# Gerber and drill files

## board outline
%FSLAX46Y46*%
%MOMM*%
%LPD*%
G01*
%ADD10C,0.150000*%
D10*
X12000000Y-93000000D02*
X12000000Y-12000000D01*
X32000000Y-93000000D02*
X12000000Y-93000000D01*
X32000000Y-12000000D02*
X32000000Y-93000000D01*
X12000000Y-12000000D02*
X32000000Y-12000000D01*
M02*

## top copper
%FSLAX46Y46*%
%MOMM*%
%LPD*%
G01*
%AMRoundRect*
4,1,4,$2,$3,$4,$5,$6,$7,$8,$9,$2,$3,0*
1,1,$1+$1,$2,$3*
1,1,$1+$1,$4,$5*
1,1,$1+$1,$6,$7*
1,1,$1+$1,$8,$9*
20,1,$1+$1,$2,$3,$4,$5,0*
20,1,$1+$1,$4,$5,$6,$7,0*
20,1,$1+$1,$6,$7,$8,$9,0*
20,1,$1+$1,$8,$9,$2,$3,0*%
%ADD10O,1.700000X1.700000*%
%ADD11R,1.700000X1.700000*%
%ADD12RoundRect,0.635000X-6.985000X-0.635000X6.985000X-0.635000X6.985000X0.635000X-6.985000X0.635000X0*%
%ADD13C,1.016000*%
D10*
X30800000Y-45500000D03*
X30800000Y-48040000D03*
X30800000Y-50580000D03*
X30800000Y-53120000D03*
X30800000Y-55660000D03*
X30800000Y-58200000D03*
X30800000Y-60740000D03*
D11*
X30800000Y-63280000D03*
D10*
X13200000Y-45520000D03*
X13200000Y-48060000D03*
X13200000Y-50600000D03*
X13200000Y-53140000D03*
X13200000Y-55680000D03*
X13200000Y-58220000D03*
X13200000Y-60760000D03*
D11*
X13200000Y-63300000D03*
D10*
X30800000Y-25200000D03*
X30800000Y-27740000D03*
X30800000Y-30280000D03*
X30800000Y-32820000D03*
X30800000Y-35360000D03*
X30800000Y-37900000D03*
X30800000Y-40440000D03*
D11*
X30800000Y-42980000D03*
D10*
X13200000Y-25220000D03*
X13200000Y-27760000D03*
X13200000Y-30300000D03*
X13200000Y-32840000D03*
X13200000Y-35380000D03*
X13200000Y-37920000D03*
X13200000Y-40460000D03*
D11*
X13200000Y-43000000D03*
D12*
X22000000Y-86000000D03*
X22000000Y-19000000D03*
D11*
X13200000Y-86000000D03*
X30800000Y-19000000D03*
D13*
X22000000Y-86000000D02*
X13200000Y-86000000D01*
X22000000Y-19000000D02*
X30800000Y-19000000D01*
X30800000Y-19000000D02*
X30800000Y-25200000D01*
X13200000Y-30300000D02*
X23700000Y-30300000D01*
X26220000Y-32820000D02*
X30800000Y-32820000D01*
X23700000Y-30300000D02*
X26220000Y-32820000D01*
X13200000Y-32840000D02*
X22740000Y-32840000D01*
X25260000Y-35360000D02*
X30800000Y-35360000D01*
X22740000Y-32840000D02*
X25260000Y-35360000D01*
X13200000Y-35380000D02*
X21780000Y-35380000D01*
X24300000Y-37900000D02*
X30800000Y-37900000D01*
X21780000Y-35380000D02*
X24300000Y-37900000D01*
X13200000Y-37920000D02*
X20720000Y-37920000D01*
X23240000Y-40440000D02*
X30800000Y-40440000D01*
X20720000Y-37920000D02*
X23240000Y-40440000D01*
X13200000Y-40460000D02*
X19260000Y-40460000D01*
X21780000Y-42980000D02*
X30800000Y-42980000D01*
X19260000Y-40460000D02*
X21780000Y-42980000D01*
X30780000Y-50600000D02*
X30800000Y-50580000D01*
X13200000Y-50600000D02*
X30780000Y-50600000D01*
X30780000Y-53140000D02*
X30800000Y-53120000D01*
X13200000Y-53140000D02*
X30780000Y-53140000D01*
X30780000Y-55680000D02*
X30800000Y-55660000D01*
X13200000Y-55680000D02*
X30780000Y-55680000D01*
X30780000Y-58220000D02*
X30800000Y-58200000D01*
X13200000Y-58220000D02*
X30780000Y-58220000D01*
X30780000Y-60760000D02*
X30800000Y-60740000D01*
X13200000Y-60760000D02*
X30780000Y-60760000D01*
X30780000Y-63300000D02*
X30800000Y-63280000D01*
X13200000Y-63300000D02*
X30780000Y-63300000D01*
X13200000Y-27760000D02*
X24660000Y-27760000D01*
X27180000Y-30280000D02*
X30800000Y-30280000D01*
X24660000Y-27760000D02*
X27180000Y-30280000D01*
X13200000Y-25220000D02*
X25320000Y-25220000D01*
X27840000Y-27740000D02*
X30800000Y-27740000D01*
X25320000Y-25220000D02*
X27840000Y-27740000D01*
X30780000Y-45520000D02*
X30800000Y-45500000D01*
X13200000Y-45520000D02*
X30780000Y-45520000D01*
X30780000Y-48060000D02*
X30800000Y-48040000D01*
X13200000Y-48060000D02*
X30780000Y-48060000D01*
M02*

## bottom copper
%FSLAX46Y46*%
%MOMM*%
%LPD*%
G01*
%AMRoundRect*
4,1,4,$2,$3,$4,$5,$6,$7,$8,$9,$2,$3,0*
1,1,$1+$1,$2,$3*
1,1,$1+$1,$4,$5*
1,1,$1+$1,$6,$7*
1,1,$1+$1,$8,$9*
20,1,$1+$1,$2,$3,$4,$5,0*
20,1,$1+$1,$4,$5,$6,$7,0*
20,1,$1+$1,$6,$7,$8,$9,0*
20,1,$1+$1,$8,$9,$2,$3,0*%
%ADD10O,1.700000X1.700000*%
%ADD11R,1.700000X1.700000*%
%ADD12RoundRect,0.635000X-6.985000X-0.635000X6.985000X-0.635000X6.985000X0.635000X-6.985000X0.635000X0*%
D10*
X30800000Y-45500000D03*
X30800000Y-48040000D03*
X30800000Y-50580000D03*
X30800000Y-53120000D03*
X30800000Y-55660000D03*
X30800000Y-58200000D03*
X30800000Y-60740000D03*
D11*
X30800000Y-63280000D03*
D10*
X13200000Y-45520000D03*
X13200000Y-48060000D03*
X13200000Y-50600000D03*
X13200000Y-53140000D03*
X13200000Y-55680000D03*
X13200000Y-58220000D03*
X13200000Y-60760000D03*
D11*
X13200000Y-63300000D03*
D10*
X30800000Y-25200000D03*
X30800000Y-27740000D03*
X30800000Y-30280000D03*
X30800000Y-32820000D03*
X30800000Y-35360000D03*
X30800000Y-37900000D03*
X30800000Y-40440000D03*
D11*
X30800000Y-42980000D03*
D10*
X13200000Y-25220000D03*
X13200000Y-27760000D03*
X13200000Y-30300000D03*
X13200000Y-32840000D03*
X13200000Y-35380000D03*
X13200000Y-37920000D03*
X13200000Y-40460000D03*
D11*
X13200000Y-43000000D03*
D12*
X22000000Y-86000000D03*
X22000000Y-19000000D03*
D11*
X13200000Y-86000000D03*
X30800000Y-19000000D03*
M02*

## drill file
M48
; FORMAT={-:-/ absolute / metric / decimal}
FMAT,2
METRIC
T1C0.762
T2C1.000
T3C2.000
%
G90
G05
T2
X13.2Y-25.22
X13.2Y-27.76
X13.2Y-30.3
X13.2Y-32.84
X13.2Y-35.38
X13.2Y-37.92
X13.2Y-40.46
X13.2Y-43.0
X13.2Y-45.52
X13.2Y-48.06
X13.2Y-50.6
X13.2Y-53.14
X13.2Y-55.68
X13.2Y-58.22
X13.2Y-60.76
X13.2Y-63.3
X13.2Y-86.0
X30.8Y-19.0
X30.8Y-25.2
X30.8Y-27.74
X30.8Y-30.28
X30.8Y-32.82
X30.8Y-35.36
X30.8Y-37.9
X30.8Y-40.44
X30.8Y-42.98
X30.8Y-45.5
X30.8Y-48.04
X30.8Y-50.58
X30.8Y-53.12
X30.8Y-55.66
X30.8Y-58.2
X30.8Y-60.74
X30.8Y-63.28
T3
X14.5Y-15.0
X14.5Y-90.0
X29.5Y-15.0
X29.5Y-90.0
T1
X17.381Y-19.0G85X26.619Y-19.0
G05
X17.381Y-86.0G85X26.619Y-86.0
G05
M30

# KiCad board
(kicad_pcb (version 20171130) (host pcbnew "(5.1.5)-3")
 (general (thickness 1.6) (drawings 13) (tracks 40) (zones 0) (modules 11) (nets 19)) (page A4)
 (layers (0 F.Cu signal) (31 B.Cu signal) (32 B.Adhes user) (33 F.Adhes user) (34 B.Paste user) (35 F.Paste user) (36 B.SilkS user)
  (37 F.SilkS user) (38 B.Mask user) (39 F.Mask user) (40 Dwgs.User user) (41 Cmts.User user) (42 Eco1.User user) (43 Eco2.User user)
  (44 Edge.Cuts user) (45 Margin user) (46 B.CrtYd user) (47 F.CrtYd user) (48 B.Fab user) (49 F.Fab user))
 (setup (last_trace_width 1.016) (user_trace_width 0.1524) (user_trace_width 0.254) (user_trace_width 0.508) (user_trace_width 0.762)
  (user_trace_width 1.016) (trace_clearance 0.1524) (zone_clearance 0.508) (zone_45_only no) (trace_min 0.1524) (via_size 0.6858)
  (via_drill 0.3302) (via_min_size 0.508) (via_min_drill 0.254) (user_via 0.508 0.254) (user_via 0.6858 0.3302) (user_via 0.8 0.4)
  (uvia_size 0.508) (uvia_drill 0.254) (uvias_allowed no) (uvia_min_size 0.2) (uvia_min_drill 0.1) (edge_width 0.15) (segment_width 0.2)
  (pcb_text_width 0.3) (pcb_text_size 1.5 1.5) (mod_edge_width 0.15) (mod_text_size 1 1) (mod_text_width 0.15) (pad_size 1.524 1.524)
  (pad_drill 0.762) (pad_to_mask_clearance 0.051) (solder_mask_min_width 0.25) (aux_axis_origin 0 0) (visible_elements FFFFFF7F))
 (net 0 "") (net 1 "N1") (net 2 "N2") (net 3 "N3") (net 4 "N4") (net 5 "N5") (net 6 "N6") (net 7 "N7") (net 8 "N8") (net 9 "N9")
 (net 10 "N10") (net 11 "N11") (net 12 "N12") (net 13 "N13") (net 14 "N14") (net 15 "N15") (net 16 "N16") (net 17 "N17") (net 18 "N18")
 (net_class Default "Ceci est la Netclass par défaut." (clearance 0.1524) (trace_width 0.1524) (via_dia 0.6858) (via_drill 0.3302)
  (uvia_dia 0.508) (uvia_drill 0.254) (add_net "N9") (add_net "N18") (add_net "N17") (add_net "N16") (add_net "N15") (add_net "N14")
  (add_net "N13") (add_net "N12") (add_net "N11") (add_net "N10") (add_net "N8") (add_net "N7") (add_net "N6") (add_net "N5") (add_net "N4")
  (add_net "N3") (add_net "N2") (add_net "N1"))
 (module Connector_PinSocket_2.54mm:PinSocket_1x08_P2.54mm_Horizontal (layer F.Cu) (at 30.8 63.28 180)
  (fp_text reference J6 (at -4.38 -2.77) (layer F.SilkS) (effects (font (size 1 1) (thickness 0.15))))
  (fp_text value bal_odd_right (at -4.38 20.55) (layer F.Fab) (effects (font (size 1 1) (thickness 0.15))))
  (pad 8 thru_hole oval (at 0 17.78 180) (size 1.7 1.7) (drill 1) (layers *.Cu *.Mask) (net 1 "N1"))
  (pad 7 thru_hole oval (at 0 15.24 180) (size 1.7 1.7) (drill 1) (layers *.Cu *.Mask) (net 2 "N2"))
  (pad 6 thru_hole oval (at 0 12.7 180) (size 1.7 1.7) (drill 1) (layers *.Cu *.Mask) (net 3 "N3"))
  (pad 5 thru_hole oval (at 0 10.16 180) (size 1.7 1.7) (drill 1) (layers *.Cu *.Mask) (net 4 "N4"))
  (pad 4 thru_hole oval (at 0 7.62 180) (size 1.7 1.7) (drill 1) (layers *.Cu *.Mask) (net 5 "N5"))
  (pad 3 thru_hole oval (at 0 5.08 180) (size 1.7 1.7) (drill 1) (layers *.Cu *.Mask) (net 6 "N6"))
  (pad 2 thru_hole oval (at 0 2.54 180) (size 1.7 1.7) (drill 1) (layers *.Cu *.Mask) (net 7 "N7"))
  (pad 1 thru_hole rect (at 0 0 180) (size 1.7 1.7) (drill 1) (layers *.Cu *.Mask) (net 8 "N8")))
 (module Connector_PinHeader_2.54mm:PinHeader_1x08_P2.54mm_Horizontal (layer F.Cu) (at 13.2 63.3 180)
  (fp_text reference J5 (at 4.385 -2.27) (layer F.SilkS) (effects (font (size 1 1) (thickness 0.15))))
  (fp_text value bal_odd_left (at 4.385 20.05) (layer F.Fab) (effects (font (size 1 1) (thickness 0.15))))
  (pad 8 thru_hole oval (at 0 17.78 180) (size 1.7 1.7) (drill 1) (layers *.Cu *.Mask) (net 1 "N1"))
  (pad 7 thru_hole oval (at 0 15.24 180) (size 1.7 1.7) (drill 1) (layers *.Cu *.Mask) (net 2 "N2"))
  (pad 6 thru_hole oval (at 0 12.7 180) (size 1.7 1.7) (drill 1) (layers *.Cu *.Mask) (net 3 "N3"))
  (pad 5 thru_hole oval (at 0 10.16 180) (size 1.7 1.7) (drill 1) (layers *.Cu *.Mask) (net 4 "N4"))
  (pad 4 thru_hole oval (at 0 7.62 180) (size 1.7 1.7) (drill 1) (layers *.Cu *.Mask) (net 5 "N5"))
  (pad 3 thru_hole oval (at 0 5.08 180) (size 1.7 1.7) (drill 1) (layers *.Cu *.Mask) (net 6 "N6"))
  (pad 2 thru_hole oval (at 0 2.54 180) (size 1.7 1.7) (drill 1) (layers *.Cu *.Mask) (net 7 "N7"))
  (pad 1 thru_hole rect (at 0 0 180) (size 1.7 1.7) (drill 1) (layers *.Cu *.Mask) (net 8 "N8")))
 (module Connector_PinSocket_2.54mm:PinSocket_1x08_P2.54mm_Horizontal (layer F.Cu) (at 30.8 42.98 180)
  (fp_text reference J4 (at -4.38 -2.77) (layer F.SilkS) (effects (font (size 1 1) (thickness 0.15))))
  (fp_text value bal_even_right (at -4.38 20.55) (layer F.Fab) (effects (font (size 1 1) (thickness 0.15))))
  (pad 8 thru_hole oval (at 0 17.78 180) (size 1.7 1.7) (drill 1) (layers *.Cu *.Mask) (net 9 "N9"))
  (pad 7 thru_hole oval (at 0 15.24 180) (size 1.7 1.7) (drill 1) (layers *.Cu *.Mask) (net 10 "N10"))
  (pad 6 thru_hole oval (at 0 12.7 180) (size 1.7 1.7) (drill 1) (layers *.Cu *.Mask) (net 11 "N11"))
  (pad 5 thru_hole oval (at 0 10.16 180) (size 1.7 1.7) (drill 1) (layers *.Cu *.Mask) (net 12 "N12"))
  (pad 4 thru_hole oval (at 0 7.62 180) (size 1.7 1.7) (drill 1) (layers *.Cu *.Mask) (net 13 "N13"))
  (pad 3 thru_hole oval (at 0 5.08 180) (size 1.7 1.7) (drill 1) (layers *.Cu *.Mask) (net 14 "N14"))
  (pad 2 thru_hole oval (at 0 2.54 180) (size 1.7 1.7) (drill 1) (layers *.Cu *.Mask) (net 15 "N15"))
  (pad 1 thru_hole rect (at 0 0 180) (size 1.7 1.7) (drill 1) (layers *.Cu *.Mask) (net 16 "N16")))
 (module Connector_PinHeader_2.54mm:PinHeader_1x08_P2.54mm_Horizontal (layer F.Cu) (at 13.2 43 180)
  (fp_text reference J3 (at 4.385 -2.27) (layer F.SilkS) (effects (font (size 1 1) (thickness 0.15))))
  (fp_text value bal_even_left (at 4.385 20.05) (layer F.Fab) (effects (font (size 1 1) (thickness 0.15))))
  (pad 8 thru_hole oval (at 0 17.78 180) (size 1.7 1.7) (drill 1) (layers *.Cu *.Mask) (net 10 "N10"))
  (pad 7 thru_hole oval (at 0 15.24 180) (size 1.7 1.7) (drill 1) (layers *.Cu *.Mask) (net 11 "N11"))
  (pad 6 thru_hole oval (at 0 12.7 180) (size 1.7 1.7) (drill 1) (layers *.Cu *.Mask) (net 12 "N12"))
  (pad 5 thru_hole oval (at 0 10.16 180) (size 1.7 1.7) (drill 1) (layers *.Cu *.Mask) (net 13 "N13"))
  (pad 4 thru_hole oval (at 0 7.62 180) (size 1.7 1.7) (drill 1) (layers *.Cu *.Mask) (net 14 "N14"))
  (pad 3 thru_hole oval (at 0 5.08 180) (size 1.7 1.7) (drill 1) (layers *.Cu *.Mask) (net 15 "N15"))
  (pad 2 thru_hole oval (at 0 2.54 180) (size 1.7 1.7) (drill 1) (layers *.Cu *.Mask) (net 16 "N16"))
  (pad 1 thru_hole rect (at 0 0 180) (size 1.7 1.7) (drill 1) (layers *.Cu *.Mask) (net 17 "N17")))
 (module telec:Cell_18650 (layer F.Cu) (at 22 19)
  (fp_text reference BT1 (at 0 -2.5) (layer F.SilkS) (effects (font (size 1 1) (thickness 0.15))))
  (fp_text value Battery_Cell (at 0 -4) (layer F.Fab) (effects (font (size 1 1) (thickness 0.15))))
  (pad 2 thru_hole roundrect (at 0 67) (size 15.24 2.54) (drill oval 10 0.762) (layers *.Cu *.Mask) (roundrect_rratio 0.25) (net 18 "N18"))
  (pad 1 thru_hole roundrect (at 0 0) (size 15.24 2.54) (drill oval 10 0.762) (layers *.Cu *.Mask) (roundrect_rratio 0.25) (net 9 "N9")))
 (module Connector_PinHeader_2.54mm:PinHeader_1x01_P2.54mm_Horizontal (layer F.Cu) (at 13.2 86 180)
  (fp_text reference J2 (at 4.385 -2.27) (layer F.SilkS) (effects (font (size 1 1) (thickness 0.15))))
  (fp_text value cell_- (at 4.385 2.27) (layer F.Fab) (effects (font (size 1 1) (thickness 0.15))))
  (pad 1 thru_hole rect (at 0 0 180) (size 1.7 1.7) (drill 1) (layers *.Cu *.Mask) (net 18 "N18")))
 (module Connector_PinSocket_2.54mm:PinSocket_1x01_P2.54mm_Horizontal (layer F.Cu) (at 30.8 19 180)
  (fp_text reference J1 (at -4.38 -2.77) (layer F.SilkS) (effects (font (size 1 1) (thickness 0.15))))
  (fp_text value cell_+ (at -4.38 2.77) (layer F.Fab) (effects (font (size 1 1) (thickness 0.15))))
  (pad 1 thru_hole rect (at 0 0 180) (size 1.7 1.7) (drill 1) (layers *.Cu *.Mask) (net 9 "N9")))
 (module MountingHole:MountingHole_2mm (layer F.Cu) (at 14.5 90)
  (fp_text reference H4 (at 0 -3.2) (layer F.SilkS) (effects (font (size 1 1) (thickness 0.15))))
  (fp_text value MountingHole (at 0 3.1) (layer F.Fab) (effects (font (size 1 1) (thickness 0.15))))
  (pad "" np_thru_hole circle (at 0 0) (size 2 2) (drill 2) (layers *.Cu *.Mask)))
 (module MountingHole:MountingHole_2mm (layer F.Cu) (at 29.5 90)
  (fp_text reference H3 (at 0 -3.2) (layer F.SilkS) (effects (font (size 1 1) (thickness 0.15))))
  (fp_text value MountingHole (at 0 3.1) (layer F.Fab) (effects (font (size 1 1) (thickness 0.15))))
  (pad "" np_thru_hole circle (at 0 0) (size 2 2) (drill 2) (layers *.Cu *.Mask)))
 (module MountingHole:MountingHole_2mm (layer F.Cu) (at 29.5 15)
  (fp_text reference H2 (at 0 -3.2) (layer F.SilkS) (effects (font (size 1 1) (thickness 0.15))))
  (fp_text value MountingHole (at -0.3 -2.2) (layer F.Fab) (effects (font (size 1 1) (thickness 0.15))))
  (pad "" np_thru_hole circle (at 0 0) (size 2 2) (drill 2) (layers *.Cu *.Mask)))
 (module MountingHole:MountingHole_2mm (layer F.Cu) (at 14.5 15)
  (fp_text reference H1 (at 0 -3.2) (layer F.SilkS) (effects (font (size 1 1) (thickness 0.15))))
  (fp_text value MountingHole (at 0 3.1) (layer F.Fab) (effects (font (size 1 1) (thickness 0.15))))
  (pad "" np_thru_hole circle (at 0 0) (size 2 2) (drill 2) (layers *.Cu *.Mask)))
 (gr_line (start 12 93) (end 12 12) (layer Edge.Cuts) (width 0.15))
 (gr_line (start 32 93) (end 12 93) (layer Edge.Cuts) (width 0.15))
 (gr_line (start 32 12) (end 32 93) (layer Edge.Cuts) (width 0.15))
 (gr_line (start 12 12) (end 32 12) (layer Edge.Cuts) (width 0.15))
 (segment (start 22 86) (end 13.2 86) (width 1.016) (layer F.Cu) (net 18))
 (segment (start 22 19) (end 30.8 19) (width 1.016) (layer F.Cu) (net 9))
 (segment (start 30.8 19) (end 30.8 25.2) (width 1.016) (layer F.Cu) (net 9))
 (segment (start 13.2 30.3) (end 23.7 30.3) (width 1.016) (layer F.Cu) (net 12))
 (segment (start 26.22 32.82) (end 30.8 32.82) (width 1.016) (layer F.Cu) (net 12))
 (segment (start 23.7 30.3) (end 26.22 32.82) (width 1.016) (layer F.Cu) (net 12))
 (segment (start 13.2 32.84) (end 22.74 32.84) (width 1.016) (layer F.Cu) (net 13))
 (segment (start 25.26 35.36) (end 30.8 35.36) (width 1.016) (layer F.Cu) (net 13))
 (segment (start 22.74 32.84) (end 25.26 35.36) (width 1.016) (layer F.Cu) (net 13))
 (segment (start 13.2 35.38) (end 21.78 35.38) (width 1.016) (layer F.Cu) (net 14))
 (segment (start 24.3 37.9) (end 30.8 37.9) (width 1.016) (layer F.Cu) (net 14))
 (segment (start 21.78 35.38) (end 24.3 37.9) (width 1.016) (layer F.Cu) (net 14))
 (segment (start 13.2 37.92) (end 20.72 37.92) (width 1.016) (layer F.Cu) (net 15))
 (segment (start 23.24 40.44) (end 30.8 40.44) (width 1.016) (layer F.Cu) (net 15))
 (segment (start 20.72 37.92) (end 23.24 40.44) (width 1.016) (layer F.Cu) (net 15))
 (segment (start 13.2 40.46) (end 19.26 40.46) (width 1.016) (layer F.Cu) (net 16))
 (segment (start 21.78 42.98) (end 30.8 42.98) (width 1.016) (layer F.Cu) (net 16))
 (segment (start 19.26 40.46) (end 21.78 42.98) (width 1.016) (layer F.Cu) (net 16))
 (segment (start 30.78 50.6) (end 30.8 50.58) (width 1.016) (layer F.Cu) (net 3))
 (segment (start 13.2 50.6) (end 30.78 50.6) (width 1.016) (layer F.Cu) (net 3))
 (segment (start 30.78 53.14) (end 30.8 53.12) (width 1.016) (layer F.Cu) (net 4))
 (segment (start 13.2 53.14) (end 30.78 53.14) (width 1.016) (layer F.Cu) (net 4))
 (segment (start 30.78 55.68) (end 30.8 55.66) (width 1.016) (layer F.Cu) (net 5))
 (segment (start 13.2 55.68) (end 30.78 55.68) (width 1.016) (layer F.Cu) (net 5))
 (segment (start 30.78 58.22) (end 30.8 58.2) (width 1.016) (layer F.Cu) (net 6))
 (segment (start 13.2 58.22) (end 30.78 58.22) (width 1.016) (layer F.Cu) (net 6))
 (segment (start 30.78 60.76) (end 30.8 60.74) (width 1.016) (layer F.Cu) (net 7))
 (segment (start 13.2 60.76) (end 30.78 60.76) (width 1.016) (layer F.Cu) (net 7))
 (segment (start 30.78 63.3) (end 30.8 63.28) (width 1.016) (layer F.Cu) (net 8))
 (segment (start 13.2 63.3) (end 30.78 63.3) (width 1.016) (layer F.Cu) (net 8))
 (segment (start 13.2 27.76) (end 24.66 27.76) (width 1.016) (layer F.Cu) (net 11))
 (segment (start 27.18 30.28) (end 30.8 30.28) (width 1.016) (layer F.Cu) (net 11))
 (segment (start 24.66 27.76) (end 27.18 30.28) (width 1.016) (layer F.Cu) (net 11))
 (segment (start 13.2 25.22) (end 25.32 25.22) (width 1.016) (layer F.Cu) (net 10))
 (segment (start 27.84 27.74) (end 30.8 27.74) (width 1.016) (layer F.Cu) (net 10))
 (segment (start 25.32 25.22) (end 27.84 27.74) (width 1.016) (layer F.Cu) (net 10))
 (segment (start 30.78 45.52) (end 30.8 45.5) (width 1.016) (layer F.Cu) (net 1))
 (segment (start 13.2 45.52) (end 30.78 45.52) (width 1.016) (layer F.Cu) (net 1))
 (segment (start 30.78 48.06) (end 30.8 48.04) (width 1.016) (layer F.Cu) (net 2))
 (segment (start 13.2 48.06) (end 30.78 48.06) (width 1.016) (layer F.Cu) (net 2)))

